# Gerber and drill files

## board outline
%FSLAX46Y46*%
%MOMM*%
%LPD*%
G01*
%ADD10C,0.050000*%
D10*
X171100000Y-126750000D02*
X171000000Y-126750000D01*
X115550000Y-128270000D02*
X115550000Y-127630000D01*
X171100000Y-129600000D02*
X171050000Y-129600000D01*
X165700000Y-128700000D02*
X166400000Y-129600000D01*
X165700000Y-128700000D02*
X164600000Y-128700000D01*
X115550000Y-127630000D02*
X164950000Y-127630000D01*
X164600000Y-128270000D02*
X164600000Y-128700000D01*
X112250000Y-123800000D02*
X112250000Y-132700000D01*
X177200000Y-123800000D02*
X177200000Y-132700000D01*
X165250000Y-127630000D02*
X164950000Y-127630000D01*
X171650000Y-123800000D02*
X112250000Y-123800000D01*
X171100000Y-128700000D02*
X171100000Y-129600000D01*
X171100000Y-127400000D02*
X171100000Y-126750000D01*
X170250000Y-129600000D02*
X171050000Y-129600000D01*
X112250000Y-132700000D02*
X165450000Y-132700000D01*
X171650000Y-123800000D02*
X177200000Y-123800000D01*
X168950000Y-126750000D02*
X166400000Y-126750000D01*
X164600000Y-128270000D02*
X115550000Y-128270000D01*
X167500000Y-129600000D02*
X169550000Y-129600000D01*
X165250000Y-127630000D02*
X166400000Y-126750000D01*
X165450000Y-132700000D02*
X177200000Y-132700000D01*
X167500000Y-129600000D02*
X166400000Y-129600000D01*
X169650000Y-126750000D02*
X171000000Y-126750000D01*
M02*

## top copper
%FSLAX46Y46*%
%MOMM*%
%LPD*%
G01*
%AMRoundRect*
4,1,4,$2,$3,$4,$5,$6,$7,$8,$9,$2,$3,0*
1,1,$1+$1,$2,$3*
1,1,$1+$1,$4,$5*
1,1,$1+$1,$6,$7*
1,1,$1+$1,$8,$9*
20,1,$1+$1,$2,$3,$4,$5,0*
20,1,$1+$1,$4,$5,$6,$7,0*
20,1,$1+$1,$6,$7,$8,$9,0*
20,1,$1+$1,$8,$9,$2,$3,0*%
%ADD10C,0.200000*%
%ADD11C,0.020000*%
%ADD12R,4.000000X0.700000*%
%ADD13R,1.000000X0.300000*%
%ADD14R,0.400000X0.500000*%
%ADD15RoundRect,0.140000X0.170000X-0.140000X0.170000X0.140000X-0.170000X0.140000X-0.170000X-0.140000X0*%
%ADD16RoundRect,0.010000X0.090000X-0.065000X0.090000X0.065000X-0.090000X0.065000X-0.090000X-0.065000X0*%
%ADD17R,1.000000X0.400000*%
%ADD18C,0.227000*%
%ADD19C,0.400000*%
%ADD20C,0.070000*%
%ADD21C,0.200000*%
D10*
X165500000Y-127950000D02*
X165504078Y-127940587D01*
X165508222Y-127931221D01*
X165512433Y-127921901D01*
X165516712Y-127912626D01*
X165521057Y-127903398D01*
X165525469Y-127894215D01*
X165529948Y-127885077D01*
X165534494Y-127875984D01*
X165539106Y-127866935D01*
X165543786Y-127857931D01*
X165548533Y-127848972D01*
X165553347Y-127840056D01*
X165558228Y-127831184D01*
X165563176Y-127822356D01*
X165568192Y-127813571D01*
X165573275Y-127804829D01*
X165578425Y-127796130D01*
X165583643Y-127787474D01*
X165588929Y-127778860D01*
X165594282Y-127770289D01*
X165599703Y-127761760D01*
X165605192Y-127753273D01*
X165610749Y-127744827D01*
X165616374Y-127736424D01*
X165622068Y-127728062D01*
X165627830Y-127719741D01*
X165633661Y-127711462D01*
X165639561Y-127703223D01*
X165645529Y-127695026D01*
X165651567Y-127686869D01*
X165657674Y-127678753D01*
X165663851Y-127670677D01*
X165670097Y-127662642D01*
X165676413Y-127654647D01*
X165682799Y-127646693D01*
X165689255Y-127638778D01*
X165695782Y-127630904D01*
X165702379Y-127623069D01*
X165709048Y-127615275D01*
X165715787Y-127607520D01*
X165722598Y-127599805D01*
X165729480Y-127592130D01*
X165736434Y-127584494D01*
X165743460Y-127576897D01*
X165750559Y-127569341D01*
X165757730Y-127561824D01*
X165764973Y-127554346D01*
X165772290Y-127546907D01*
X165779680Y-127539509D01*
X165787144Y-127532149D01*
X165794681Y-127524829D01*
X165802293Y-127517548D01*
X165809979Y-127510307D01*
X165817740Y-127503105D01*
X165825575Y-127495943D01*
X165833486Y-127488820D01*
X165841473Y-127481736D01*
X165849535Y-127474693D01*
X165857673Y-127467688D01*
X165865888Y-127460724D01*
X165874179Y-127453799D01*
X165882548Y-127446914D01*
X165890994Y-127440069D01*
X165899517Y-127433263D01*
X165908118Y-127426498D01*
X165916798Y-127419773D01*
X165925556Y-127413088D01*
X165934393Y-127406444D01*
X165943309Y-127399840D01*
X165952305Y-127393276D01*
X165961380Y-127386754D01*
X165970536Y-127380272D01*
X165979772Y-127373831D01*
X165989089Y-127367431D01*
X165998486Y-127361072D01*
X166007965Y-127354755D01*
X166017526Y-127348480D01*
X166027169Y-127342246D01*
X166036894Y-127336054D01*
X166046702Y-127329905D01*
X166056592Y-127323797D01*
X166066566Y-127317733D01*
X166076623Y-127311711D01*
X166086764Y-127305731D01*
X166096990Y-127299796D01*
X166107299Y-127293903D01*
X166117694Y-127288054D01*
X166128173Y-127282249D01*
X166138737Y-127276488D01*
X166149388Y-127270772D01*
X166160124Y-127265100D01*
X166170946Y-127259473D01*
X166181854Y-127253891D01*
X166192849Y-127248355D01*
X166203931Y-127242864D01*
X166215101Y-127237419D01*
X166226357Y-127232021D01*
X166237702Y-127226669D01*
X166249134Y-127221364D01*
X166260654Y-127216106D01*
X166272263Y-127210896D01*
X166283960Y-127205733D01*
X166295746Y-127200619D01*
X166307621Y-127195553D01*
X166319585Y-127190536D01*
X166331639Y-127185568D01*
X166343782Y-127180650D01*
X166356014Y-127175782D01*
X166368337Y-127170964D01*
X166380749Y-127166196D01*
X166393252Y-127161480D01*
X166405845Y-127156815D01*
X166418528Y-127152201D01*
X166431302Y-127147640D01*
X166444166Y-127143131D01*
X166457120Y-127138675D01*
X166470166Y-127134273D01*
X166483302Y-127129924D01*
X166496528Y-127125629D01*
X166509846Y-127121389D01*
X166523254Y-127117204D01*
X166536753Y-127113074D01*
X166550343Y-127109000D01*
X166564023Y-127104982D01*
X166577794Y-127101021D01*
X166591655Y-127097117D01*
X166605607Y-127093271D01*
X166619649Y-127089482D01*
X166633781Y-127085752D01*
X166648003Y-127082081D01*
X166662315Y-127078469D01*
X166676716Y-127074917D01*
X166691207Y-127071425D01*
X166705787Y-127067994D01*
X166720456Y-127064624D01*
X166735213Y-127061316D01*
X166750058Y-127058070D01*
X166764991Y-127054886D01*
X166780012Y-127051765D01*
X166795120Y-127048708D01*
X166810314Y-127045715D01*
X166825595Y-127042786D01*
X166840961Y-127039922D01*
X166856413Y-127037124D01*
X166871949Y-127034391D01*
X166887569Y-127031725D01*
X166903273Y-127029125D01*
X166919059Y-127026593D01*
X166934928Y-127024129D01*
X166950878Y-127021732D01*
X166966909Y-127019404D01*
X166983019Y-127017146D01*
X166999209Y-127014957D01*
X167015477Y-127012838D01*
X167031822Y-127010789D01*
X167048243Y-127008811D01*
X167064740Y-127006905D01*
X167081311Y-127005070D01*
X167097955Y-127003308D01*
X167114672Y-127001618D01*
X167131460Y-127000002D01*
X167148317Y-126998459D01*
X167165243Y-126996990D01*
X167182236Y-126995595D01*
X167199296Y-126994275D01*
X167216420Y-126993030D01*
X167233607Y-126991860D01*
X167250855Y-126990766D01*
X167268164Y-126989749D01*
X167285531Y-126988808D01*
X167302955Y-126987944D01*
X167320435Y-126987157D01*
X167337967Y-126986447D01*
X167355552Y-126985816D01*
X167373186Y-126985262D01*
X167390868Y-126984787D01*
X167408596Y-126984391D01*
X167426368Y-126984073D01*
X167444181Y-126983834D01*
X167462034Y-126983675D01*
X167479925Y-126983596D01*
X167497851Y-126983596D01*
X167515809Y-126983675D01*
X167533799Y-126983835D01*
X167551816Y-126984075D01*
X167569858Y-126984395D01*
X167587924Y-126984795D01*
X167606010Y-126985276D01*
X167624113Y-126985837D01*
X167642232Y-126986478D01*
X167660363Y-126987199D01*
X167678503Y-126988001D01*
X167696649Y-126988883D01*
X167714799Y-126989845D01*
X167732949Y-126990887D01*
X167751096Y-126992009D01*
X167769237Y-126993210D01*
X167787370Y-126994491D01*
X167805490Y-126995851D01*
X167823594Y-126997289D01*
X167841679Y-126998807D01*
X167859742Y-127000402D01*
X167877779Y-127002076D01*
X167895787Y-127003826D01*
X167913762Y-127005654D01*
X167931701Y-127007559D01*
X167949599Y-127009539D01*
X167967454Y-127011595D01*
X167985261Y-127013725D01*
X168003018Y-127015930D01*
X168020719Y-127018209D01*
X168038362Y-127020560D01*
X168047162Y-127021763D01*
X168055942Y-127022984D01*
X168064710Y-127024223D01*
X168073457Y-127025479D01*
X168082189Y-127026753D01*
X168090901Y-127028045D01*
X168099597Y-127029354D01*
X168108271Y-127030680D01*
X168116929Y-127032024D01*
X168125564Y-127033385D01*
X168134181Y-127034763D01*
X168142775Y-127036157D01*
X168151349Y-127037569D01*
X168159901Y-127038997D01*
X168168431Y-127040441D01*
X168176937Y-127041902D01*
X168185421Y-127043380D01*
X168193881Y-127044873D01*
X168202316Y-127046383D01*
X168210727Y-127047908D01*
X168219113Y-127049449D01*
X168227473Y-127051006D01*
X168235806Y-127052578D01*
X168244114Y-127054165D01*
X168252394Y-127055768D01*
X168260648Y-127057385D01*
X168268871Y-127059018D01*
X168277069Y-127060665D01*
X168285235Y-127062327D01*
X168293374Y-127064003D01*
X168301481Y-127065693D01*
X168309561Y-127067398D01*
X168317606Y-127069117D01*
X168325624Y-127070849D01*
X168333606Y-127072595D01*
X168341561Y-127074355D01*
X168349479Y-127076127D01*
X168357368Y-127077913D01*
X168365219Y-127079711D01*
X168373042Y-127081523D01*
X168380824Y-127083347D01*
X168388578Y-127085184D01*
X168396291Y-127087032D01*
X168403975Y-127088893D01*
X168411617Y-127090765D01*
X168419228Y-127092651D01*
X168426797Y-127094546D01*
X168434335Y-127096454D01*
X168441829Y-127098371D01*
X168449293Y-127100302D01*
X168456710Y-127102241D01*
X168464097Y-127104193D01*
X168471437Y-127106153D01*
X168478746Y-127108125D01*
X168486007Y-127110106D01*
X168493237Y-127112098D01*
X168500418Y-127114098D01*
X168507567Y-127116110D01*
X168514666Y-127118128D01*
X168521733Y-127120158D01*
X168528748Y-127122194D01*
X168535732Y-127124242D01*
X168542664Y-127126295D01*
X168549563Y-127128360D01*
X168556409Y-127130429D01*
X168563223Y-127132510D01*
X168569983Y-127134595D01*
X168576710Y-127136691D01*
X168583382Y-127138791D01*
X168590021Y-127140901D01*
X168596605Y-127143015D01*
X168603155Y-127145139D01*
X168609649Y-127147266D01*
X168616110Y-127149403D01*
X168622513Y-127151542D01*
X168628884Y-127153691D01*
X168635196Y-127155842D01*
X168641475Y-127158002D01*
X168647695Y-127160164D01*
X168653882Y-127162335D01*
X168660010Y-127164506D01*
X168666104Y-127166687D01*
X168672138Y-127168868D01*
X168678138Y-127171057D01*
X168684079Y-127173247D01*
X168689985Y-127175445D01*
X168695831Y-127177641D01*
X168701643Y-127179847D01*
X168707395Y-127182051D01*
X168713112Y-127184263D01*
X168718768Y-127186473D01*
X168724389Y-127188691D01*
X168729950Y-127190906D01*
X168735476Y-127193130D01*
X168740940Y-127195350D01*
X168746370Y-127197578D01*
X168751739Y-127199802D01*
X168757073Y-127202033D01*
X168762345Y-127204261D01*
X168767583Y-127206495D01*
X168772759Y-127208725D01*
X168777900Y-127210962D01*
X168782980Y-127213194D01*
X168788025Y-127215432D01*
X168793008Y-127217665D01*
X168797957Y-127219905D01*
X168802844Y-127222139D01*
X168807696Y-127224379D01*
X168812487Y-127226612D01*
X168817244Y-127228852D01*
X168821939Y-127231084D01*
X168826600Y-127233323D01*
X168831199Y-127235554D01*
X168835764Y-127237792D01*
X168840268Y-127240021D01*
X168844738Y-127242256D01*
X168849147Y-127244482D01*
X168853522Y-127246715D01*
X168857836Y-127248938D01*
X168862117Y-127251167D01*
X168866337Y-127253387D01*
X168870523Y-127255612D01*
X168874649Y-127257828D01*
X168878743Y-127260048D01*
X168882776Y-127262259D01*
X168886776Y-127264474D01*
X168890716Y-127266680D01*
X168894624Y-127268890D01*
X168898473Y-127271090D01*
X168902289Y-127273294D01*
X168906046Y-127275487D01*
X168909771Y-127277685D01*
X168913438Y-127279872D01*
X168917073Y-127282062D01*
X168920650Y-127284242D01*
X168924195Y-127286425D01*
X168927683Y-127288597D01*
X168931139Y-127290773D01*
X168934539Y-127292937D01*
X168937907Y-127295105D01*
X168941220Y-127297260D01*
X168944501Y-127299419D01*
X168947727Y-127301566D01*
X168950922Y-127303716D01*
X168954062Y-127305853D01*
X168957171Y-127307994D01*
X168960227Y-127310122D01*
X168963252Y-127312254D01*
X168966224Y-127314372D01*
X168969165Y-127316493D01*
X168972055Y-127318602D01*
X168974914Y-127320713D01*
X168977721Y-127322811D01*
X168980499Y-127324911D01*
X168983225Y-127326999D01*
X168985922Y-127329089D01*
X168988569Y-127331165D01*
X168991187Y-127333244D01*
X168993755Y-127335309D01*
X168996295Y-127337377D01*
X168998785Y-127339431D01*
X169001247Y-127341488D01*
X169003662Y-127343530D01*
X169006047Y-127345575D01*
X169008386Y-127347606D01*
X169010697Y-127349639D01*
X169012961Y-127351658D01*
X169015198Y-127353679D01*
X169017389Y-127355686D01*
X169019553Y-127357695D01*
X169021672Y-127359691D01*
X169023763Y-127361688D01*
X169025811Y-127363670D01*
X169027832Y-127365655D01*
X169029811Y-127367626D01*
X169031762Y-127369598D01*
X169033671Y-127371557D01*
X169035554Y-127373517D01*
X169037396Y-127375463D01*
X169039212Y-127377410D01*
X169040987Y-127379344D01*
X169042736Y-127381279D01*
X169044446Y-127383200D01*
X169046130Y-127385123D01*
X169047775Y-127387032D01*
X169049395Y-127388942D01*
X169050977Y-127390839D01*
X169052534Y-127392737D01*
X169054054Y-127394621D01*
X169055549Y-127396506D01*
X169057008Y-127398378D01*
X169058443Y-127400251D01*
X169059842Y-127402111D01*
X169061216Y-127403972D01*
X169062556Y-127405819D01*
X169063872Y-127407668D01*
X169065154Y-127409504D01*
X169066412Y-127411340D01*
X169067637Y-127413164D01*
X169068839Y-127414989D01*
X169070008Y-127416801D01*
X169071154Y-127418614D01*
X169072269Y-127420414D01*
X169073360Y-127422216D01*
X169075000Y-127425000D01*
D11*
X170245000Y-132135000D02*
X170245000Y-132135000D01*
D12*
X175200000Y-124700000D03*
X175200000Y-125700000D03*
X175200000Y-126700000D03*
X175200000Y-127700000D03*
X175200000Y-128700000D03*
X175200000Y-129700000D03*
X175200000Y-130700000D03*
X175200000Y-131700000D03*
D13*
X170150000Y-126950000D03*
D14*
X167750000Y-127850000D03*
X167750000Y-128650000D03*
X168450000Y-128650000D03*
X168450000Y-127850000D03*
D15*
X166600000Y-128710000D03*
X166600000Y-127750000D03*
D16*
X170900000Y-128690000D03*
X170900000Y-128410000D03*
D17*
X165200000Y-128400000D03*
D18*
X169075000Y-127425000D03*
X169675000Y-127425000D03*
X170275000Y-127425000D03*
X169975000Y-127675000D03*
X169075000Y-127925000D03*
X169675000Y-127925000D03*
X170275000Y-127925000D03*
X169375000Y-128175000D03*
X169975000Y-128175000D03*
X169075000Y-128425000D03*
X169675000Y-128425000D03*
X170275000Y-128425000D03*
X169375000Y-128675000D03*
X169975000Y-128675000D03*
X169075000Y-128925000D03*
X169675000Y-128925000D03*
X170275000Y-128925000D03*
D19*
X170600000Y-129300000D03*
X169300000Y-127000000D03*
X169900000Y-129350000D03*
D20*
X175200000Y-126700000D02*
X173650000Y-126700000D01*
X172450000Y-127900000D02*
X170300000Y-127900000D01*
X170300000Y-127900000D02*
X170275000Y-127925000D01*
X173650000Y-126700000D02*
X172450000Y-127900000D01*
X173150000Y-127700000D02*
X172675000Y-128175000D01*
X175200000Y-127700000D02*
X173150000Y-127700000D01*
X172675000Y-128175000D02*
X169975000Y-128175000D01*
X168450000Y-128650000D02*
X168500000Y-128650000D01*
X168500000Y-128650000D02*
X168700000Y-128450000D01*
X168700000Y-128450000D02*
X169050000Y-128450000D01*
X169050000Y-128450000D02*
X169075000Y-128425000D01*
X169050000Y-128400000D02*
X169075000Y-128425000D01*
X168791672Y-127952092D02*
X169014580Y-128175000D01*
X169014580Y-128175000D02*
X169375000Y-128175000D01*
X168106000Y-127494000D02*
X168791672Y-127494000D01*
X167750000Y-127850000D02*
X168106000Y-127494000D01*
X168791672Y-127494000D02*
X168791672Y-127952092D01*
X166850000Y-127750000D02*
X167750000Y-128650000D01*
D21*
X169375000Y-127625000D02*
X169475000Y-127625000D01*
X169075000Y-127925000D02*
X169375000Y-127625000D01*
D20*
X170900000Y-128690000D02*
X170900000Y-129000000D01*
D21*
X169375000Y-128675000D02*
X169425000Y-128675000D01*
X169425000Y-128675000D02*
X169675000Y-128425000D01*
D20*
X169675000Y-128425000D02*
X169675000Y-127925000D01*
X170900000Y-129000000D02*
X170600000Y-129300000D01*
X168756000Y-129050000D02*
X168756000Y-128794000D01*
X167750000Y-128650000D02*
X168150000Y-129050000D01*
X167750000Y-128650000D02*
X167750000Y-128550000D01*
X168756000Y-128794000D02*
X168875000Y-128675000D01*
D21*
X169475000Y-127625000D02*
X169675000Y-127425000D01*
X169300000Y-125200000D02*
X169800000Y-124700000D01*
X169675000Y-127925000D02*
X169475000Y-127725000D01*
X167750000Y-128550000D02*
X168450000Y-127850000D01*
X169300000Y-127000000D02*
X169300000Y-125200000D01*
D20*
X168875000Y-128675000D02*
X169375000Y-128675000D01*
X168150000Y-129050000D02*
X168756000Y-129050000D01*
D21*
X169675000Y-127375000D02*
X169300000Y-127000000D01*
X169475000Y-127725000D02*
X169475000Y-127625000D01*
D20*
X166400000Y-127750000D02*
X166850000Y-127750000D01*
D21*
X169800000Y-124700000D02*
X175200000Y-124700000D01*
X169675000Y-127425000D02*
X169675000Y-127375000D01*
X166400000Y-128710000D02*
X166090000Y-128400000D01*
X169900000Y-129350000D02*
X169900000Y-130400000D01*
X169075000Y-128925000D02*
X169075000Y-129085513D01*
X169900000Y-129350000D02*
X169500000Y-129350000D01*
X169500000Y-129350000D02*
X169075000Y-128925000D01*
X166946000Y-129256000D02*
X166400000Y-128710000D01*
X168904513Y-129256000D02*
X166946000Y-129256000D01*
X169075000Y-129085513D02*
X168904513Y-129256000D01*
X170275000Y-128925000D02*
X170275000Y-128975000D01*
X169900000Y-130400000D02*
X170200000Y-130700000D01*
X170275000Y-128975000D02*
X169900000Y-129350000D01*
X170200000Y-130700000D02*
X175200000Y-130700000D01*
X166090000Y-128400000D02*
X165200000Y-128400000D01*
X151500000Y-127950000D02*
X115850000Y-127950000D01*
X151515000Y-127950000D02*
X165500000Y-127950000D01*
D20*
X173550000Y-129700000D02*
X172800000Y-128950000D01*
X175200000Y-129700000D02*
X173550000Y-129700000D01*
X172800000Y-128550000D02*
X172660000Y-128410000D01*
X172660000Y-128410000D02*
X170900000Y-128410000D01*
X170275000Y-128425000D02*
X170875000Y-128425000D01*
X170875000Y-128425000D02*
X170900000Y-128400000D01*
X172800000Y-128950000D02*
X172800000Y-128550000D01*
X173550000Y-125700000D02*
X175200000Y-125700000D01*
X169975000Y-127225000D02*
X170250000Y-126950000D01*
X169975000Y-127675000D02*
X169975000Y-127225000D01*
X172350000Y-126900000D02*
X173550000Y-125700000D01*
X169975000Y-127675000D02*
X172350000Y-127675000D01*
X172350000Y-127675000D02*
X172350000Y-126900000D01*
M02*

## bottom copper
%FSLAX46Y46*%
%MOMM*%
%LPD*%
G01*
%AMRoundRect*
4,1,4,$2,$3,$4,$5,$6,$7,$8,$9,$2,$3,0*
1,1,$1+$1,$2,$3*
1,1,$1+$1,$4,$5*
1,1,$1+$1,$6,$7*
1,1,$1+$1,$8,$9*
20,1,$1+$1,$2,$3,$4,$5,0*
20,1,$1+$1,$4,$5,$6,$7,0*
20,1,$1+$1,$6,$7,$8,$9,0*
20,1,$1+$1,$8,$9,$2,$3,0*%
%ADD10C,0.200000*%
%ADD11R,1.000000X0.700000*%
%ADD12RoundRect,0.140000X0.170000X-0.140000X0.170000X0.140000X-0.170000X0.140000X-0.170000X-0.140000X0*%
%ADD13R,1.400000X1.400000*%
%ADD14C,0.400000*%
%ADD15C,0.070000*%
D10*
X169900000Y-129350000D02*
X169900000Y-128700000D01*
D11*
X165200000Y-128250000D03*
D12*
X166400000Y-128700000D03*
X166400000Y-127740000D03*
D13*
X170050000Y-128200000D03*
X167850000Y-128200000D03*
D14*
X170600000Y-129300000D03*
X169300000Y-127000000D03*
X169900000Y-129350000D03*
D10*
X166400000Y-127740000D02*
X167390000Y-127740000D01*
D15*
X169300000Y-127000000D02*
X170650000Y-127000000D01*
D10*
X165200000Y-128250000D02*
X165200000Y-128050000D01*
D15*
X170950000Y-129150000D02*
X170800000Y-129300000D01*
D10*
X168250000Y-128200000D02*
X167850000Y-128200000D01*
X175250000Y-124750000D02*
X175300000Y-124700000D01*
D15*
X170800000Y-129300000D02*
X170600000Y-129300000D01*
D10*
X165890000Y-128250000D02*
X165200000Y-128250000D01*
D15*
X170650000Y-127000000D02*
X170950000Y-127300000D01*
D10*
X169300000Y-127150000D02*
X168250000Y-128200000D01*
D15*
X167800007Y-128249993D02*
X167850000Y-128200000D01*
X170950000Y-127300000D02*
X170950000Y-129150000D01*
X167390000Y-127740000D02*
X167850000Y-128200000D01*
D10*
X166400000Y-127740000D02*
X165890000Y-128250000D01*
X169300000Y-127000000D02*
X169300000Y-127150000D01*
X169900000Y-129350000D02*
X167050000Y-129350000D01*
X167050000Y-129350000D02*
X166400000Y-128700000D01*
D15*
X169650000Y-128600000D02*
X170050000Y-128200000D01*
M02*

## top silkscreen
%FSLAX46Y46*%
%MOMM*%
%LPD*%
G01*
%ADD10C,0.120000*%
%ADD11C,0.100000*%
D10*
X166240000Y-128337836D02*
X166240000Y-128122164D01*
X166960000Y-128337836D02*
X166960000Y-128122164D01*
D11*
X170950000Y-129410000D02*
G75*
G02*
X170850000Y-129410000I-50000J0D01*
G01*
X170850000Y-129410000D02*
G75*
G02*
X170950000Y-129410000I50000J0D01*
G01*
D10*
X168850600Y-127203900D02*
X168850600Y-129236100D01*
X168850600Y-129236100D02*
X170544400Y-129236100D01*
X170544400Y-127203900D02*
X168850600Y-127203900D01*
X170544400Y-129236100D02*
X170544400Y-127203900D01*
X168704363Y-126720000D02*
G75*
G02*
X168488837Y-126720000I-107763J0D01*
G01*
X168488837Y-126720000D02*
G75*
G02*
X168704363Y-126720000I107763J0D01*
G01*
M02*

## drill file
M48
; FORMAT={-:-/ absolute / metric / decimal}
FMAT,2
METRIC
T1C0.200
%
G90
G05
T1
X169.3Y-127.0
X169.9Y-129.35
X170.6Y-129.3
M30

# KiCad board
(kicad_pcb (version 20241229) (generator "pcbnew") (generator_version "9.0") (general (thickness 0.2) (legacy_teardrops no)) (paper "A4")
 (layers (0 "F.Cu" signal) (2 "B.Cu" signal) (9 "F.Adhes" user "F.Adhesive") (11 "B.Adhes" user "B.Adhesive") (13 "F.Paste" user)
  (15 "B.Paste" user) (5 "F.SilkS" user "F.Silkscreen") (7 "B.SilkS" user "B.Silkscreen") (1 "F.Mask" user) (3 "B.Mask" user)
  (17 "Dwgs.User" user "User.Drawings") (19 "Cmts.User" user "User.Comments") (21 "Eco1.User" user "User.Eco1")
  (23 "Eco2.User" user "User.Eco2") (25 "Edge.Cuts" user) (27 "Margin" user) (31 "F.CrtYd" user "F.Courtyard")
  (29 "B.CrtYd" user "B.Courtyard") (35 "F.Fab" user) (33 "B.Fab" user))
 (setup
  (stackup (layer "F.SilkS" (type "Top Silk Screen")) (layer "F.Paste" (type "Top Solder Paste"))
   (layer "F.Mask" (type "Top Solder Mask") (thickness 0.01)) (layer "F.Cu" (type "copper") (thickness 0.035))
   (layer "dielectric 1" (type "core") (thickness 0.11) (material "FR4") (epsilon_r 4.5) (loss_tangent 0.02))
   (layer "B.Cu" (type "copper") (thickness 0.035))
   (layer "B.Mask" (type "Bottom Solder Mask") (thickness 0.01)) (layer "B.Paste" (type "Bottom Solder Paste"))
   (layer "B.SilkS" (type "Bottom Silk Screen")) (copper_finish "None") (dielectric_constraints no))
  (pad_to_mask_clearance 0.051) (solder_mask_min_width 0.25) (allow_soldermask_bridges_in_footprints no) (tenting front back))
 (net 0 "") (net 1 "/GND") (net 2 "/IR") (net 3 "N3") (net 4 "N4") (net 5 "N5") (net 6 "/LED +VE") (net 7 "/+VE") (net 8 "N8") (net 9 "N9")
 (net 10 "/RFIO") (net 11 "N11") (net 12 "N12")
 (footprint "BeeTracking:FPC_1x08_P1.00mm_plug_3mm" (layer "F.Cu") (at 173.2 128.2)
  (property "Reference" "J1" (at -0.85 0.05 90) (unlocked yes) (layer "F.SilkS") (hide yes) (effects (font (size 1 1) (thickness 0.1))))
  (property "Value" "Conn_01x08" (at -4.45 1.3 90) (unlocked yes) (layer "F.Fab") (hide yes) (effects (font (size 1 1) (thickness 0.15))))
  (pad "1" connect rect (at 2 -3.5) (size 4 0.7) (layers "F.Cu" "F.Mask") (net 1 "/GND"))
  (pad "2" connect rect (at 2 -2.5) (size 4 0.7) (layers "F.Cu" "F.Mask") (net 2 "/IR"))
  (pad "3" connect rect (at 2 -1.5) (size 4 0.7) (layers "F.Cu" "F.Mask") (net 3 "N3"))
  (pad "4" connect rect (at 2 -0.5) (size 4 0.7) (layers "F.Cu" "F.Mask") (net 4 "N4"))
  (pad "5" connect rect (at 2 0.5) (size 4 0.7) (layers "F.Cu" "F.Mask") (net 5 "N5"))
  (pad "6" connect rect (at 2 1.5) (size 4 0.7) (layers "F.Cu" "F.Mask") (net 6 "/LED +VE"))
  (pad "7" connect rect (at 2 2.5) (size 4 0.7) (layers "F.Cu" "F.Mask") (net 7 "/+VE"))
  (pad "8" connect rect (at 2 3.5) (size 4 0.7) (layers "F.Cu" "F.Mask")))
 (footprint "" (layer "F.Cu") (at 170.35 126.1)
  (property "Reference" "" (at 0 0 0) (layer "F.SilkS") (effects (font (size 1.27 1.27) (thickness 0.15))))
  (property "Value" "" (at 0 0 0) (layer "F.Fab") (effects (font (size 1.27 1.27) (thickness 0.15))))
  (pad "1" smd rect (at -0.2 0.85) (size 1 0.3) (layers "F.Cu" "F.Mask") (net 2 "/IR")))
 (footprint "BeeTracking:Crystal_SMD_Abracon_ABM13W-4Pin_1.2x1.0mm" (layer "F.Cu") (at 168.1 128.25 -90)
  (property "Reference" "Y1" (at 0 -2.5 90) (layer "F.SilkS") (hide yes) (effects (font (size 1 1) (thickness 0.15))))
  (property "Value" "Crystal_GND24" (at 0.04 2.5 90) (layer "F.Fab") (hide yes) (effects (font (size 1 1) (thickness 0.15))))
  (pad "1" smd rect (at -0.4 0.35 270) (size 0.5 0.4) (layers "F.Cu" "F.Mask" "F.Paste") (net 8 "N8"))
  (pad "2" smd rect (at 0.4 0.35 270) (size 0.5 0.4) (layers "F.Cu" "F.Mask" "F.Paste") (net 1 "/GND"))
  (pad "3" smd rect (at 0.4 -0.35 270) (size 0.5 0.4) (layers "F.Cu" "F.Mask" "F.Paste") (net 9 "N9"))
  (pad "4" smd rect (at -0.4 -0.35 270) (size 0.5 0.4) (layers "F.Cu" "F.Mask" "F.Paste") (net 1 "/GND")))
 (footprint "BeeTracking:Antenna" (layer "F.Cu") (at 170.245 132.135)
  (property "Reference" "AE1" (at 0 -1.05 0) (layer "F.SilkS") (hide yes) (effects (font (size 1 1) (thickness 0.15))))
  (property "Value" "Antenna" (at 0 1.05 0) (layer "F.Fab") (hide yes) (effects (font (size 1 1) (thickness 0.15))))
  (fp_line (start 0 0) (end 0 0) (stroke (width 0.02) (type solid)) (layer "F.Cu")))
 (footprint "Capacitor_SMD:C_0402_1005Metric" (layer "F.Cu") (at 166.6 128.23 90)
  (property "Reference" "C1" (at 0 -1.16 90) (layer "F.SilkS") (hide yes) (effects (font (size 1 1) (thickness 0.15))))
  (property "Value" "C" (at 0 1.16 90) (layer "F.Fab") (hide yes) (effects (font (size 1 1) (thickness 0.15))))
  (fp_line (start -0.107836 -0.36) (end 0.107836 -0.36) (stroke (width 0.12) (type solid)) (layer "F.SilkS"))
  (fp_line (start -0.107836 0.36) (end 0.107836 0.36) (stroke (width 0.12) (type solid)) (layer "F.SilkS"))
  (pad "1" smd roundrect (at -0.48 0 90) (size 0.56 0.62) (layers "F.Cu" "F.Mask" "F.Paste") (roundrect_rratio 0.25) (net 7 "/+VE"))
  (pad "2" smd roundrect (at 0.48 0 90) (size 0.56 0.62) (layers "F.Cu" "F.Mask" "F.Paste") (roundrect_rratio 0.25) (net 1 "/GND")))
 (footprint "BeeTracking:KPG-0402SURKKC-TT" (layer "F.Cu") (at 170.9 128.55 90)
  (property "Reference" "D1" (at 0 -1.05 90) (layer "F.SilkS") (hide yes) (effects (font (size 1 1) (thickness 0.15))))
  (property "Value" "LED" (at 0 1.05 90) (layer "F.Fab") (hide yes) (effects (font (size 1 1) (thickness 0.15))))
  (fp_circle (center -0.86 0) (end -0.81 0) (stroke (width 0.1) (type solid)) (fill no) (layer "F.SilkS"))
  (pad "" smd roundrect (at -0.14 0 90) (size 0.15 0.2) (layers "F.Mask") (roundrect_rratio 0.06666666667))
  (pad "" smd roundrect (at -0.1225 0 90) (size 0.1 0.17) (layers "F.Paste") (roundrect_rratio 0.25))
  (pad "" smd roundrect (at 0.1225 0 90) (size 0.1 0.17) (layers "F.Paste") (roundrect_rratio 0.25))
  (pad "" smd roundrect (at 0.14 0 90) (size 0.15 0.2) (layers "F.Mask") (roundrect_rratio 0.06666666667))
  (pad "1" smd roundrect (at -0.14 0 90) (size 0.15 0.2) (layers "F.Cu" "F.Mask") (roundrect_rratio 0.06666666667) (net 1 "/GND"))
  (pad "2" smd roundrect (at 0.14 0 90) (size 0.15 0.2) (layers "F.Cu" "F.Mask") (roundrect_rratio 0.06666666667) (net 6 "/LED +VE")))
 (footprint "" (layer "F.Cu") (at 165.4 127.6)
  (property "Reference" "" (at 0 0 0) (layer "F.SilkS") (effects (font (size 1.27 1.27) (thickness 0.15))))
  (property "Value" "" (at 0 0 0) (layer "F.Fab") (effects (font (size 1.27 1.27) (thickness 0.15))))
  (pad "1" smd rect (at -0.2 0.8) (size 1 0.4) (layers "F.Cu" "F.Mask") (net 7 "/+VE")))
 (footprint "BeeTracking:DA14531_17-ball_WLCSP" (layer "F.Cu") (at 169.697 128.22)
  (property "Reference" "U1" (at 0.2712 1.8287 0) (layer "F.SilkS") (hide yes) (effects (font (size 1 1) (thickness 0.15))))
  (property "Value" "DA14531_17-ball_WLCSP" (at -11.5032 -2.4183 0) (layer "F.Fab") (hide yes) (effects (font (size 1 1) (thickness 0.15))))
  (fp_line (start -0.8464 -1.0161) (end -0.8464 1.0161) (stroke (width 0.12) (type solid)) (layer "F.SilkS"))
  (fp_line (start -0.8464 1.0161) (end 0.8474 1.0161) (stroke (width 0.12) (type solid)) (layer "F.SilkS"))
  (fp_line (start 0.8474 -1.0161) (end -0.8464 -1.0161) (stroke (width 0.12) (type solid)) (layer "F.SilkS"))
  (fp_line (start 0.8474 1.0161) (end 0.8474 -1.0161) (stroke (width 0.12) (type solid)) (layer "F.SilkS"))
  (fp_circle (center -1.1004 -1.5) (end -1.0242 -1.4238) (stroke (width 0.12) (type solid)) (fill no) (layer "F.SilkS"))
  (pad "A1" smd circle (at -0.622 -0.795) (size 0.227 0.227) (layers "F.Cu" "F.Mask" "F.Paste") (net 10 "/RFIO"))
  (pad "A3" smd circle (at -0.022 -0.795) (size 0.227 0.227) (layers "F.Cu" "F.Mask" "F.Paste") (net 1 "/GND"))
  (pad "A5" smd circle (at 0.578 -0.795) (size 0.227 0.227) (layers "F.Cu" "F.Mask" "F.Paste") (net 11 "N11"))
  (pad "B4" smd circle (at 0.278 -0.545) (size 0.227 0.227) (layers "F.Cu" "F.Mask" "F.Paste") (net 2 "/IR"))
  (pad "C1" smd circle (at -0.622 -0.295) (size 0.227 0.227) (layers "F.Cu" "F.Mask" "F.Paste") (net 1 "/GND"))
  (pad "C3" smd circle (at -0.022 -0.295) (size 0.227 0.227) (layers "F.Cu" "F.Mask" "F.Paste") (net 1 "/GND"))
  (pad "C5" smd circle (at 0.578 -0.295) (size 0.227 0.227) (layers "F.Cu" "F.Mask" "F.Paste") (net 3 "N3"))
  (pad "D2" smd circle (at -0.322 -0.045) (size 0.227 0.227) (layers "F.Cu" "F.Mask" "F.Paste") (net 8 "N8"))
  (pad "D4" smd circle (at 0.278 -0.045) (size 0.227 0.227) (layers "F.Cu" "F.Mask" "F.Paste") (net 4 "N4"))
  (pad "E1" smd circle (at -0.622 0.205) (size 0.227 0.227) (layers "F.Cu" "F.Mask" "F.Paste") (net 9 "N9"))
  (pad "E3" smd circle (at -0.022 0.205) (size 0.227 0.227) (layers "F.Cu" "F.Mask" "F.Paste") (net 1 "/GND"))
  (pad "E5" smd circle (at 0.578 0.205) (size 0.227 0.227) (layers "F.Cu" "F.Mask" "F.Paste") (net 6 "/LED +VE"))
  (pad "F2" smd circle (at -0.322 0.455) (size 0.227 0.227) (layers "F.Cu" "F.Mask" "F.Paste") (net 1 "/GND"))
  (pad "F4" smd circle (at 0.278 0.455) (size 0.227 0.227) (layers "F.Cu" "F.Mask" "F.Paste") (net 5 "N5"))
  (pad "G1" smd circle (at -0.622 0.705) (size 0.227 0.227) (layers "F.Cu" "F.Mask" "F.Paste") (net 7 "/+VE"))
  (pad "G3" smd circle (at -0.022 0.705) (size 0.227 0.227) (layers "F.Cu" "F.Mask" "F.Paste") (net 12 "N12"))
  (pad "G5" smd circle (at 0.578 0.705) (size 0.227 0.227) (layers "F.Cu" "F.Mask" "F.Paste") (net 7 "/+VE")))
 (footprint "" (layer "B.Cu") (at 165.2 128.4 180)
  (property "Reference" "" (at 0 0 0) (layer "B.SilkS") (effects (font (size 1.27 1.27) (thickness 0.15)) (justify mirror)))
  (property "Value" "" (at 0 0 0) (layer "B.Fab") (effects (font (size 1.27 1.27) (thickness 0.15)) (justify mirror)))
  (pad "1" smd rect (at 0 0.15 180) (size 1 0.7) (layers "B.Cu" "B.Mask") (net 1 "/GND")))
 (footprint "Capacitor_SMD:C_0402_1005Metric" (layer "B.Cu") (at 166.4 128.22 90)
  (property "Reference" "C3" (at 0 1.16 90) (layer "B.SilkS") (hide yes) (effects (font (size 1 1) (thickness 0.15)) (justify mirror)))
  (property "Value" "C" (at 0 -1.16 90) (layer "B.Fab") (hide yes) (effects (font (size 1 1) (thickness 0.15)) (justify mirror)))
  (pad "1" smd roundrect (at -0.48 0 90) (size 0.56 0.62) (layers "B.Cu" "B.Mask" "B.Paste") (roundrect_rratio 0.25) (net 7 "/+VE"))
  (pad "2" smd roundrect (at 0.48 0 90) (size 0.56 0.62) (layers "B.Cu" "B.Mask" "B.Paste") (roundrect_rratio 0.25) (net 1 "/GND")))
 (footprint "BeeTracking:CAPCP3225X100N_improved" (layer "B.Cu") (at 168.95 128.2 180)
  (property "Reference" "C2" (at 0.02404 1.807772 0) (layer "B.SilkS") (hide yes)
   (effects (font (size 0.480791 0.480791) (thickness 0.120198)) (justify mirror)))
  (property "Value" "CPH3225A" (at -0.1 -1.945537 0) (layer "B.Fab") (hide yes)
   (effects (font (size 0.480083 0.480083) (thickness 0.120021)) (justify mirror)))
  (pad "1" smd rect (at -1.1 0) (size 1.4 1.4) (layers "B.Cu" "B.Mask" "B.Paste") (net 7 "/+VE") (solder_mask_margin 0.102))
  (pad "2" smd rect (at 1.1 0) (size 1.4 1.4) (layers "B.Cu" "B.Mask" "B.Paste") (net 1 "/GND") (solder_mask_margin 0.102)))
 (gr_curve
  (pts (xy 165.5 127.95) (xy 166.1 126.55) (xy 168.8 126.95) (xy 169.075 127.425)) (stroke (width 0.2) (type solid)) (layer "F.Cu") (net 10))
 (gr_line (start 169.9 129.35) (end 169.9 128.7) (stroke (width 0.2) (type default)) (layer "B.Cu") (net 7))
 (gr_line (start 171.1 126.75) (end 171 126.75) (stroke (width 0.05) (type default)) (layer "Edge.Cuts"))
 (gr_line (start 115.55 128.27) (end 115.55 127.63) (stroke (width 0.05) (type default)) (layer "Edge.Cuts"))
 (gr_line (start 171.1 129.6) (end 171.05 129.6) (stroke (width 0.05) (type default)) (layer "Edge.Cuts"))
 (gr_line (start 165.7 128.7) (end 166.4 129.6) (stroke (width 0.05) (type default)) (layer "Edge.Cuts"))
 (gr_line (start 165.7 128.7) (end 164.6 128.7) (stroke (width 0.05) (type default)) (layer "Edge.Cuts"))
 (gr_line (start 115.55 127.63) (end 164.95 127.63) (stroke (width 0.05) (type default)) (layer "Edge.Cuts"))
 (gr_line (start 164.6 128.27) (end 164.6 128.7) (stroke (width 0.05) (type default)) (layer "Edge.Cuts"))
 (gr_line (start 112.25 123.8) (end 112.25 132.7) (stroke (width 0.05) (type default)) (layer "Edge.Cuts"))
 (gr_line (start 177.2 123.8) (end 177.2 132.7) (stroke (width 0.05) (type default)) (layer "Edge.Cuts"))
 (gr_line (start 165.25 127.63) (end 164.95 127.63) (stroke (width 0.05) (type default)) (layer "Edge.Cuts"))
 (gr_line (start 171.65 123.8) (end 112.25 123.8) (stroke (width 0.05) (type default)) (layer "Edge.Cuts"))
 (gr_line (start 171.1 128.7) (end 171.1 129.6) (stroke (width 0.05) (type default)) (layer "Edge.Cuts"))
 (gr_line (start 171.1 127.4) (end 171.1 126.75) (stroke (width 0.05) (type default)) (layer "Edge.Cuts"))
 (gr_line (start 170.25 129.6) (end 171.05 129.6) (stroke (width 0.05) (type default)) (layer "Edge.Cuts"))
 (gr_line (start 112.25 132.7) (end 165.45 132.7) (stroke (width 0.05) (type default)) (layer "Edge.Cuts"))
 (gr_line (start 171.65 123.8) (end 177.2 123.8) (stroke (width 0.05) (type default)) (layer "Edge.Cuts"))
 (gr_line (start 168.95 126.75) (end 166.4 126.75) (stroke (width 0.05) (type default)) (layer "Edge.Cuts"))
 (gr_line (start 164.6 128.27) (end 115.55 128.27) (stroke (width 0.05) (type default)) (layer "Edge.Cuts"))
 (gr_line (start 167.5 129.6) (end 169.55 129.6) (stroke (width 0.05) (type default)) (layer "Edge.Cuts"))
 (gr_line (start 165.25 127.63) (end 166.4 126.75) (stroke (width 0.05) (type default)) (layer "Edge.Cuts"))
 (gr_line (start 165.45 132.7) (end 177.2 132.7) (stroke (width 0.05) (type default)) (layer "Edge.Cuts"))
 (gr_line (start 167.5 129.6) (end 166.4 129.6) (stroke (width 0.05) (type default)) (layer "Edge.Cuts"))
 (gr_line (start 169.65 126.75) (end 171 126.75) (stroke (width 0.05) (type default)) (layer "Edge.Cuts"))
 (segment (start 175.2 126.7) (end 173.65 126.7) (width 0.07) (layer "F.Cu") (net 3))
 (segment (start 172.45 127.9) (end 170.3 127.9) (width 0.07) (layer "F.Cu") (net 3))
 (segment (start 170.3 127.9) (end 170.275 127.925) (width 0.07) (layer "F.Cu") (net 3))
 (segment (start 173.65 126.7) (end 172.45 127.9) (width 0.07) (layer "F.Cu") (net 3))
 (segment (start 173.15 127.7) (end 172.675 128.175) (width 0.07) (layer "F.Cu") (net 4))
 (segment (start 175.2 127.7) (end 173.15 127.7) (width 0.07) (layer "F.Cu") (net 4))
 (segment (start 172.675 128.175) (end 169.975 128.175) (width 0.07) (layer "F.Cu") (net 4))
 (segment (start 168.45 128.65) (end 168.5 128.65) (width 0.07) (layer "F.Cu") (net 9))
 (segment (start 168.5 128.65) (end 168.7 128.45) (width 0.07) (layer "F.Cu") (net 9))
 (segment (start 168.7 128.45) (end 169.05 128.45) (width 0.07) (layer "F.Cu") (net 9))
 (segment (start 169.05 128.45) (end 169.075 128.425) (width 0.07) (layer "F.Cu") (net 9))
 (segment (start 169.05 128.4) (end 169.075 128.425) (width 0.07) (layer "F.Cu") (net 9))
 (segment (start 168.791672 127.952092) (end 169.01458 128.175) (width 0.07) (layer "F.Cu") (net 8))
 (segment (start 169.01458 128.175) (end 169.375 128.175) (width 0.07) (layer "F.Cu") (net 8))
 (segment (start 168.106 127.494) (end 168.791672 127.494) (width 0.07) (layer "F.Cu") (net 8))
 (segment (start 167.75 127.85) (end 168.106 127.494) (width 0.07) (layer "F.Cu") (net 8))
 (segment (start 168.791672 127.494) (end 168.791672 127.952092) (width 0.07) (layer "F.Cu") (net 8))
 (segment (start 166.85 127.75) (end 167.75 128.65) (width 0.07) (layer "F.Cu") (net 1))
 (segment (start 169.375 127.625) (end 169.475 127.625) (width 0.2) (layer "F.Cu") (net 1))
 (segment (start 169.075 127.925) (end 169.375 127.625) (width 0.2) (layer "F.Cu") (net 1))
 (segment (start 170.9 128.69) (end 170.9 129) (width 0.07) (layer "F.Cu") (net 1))
 (segment (start 169.375 128.675) (end 169.425 128.675) (width 0.2) (layer "F.Cu") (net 1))
 (segment (start 169.425 128.675) (end 169.675 128.425) (width 0.2) (layer "F.Cu") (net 1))
 (segment (start 169.675 128.425) (end 169.675 127.925) (width 0.07) (layer "F.Cu") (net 1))
 (segment (start 170.9 129) (end 170.6 129.3) (width 0.07) (layer "F.Cu") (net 1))
 (segment (start 168.756 129.05) (end 168.756 128.794) (width 0.07) (layer "F.Cu") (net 1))
 (segment (start 167.75 128.65) (end 168.15 129.05) (width 0.07) (layer "F.Cu") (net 1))
 (segment (start 167.75 128.65) (end 167.75 128.55) (width 0.07) (layer "F.Cu") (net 1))
 (segment (start 168.756 128.794) (end 168.875 128.675) (width 0.07) (layer "F.Cu") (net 1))
 (segment (start 169.475 127.625) (end 169.675 127.425) (width 0.2) (layer "F.Cu") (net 1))
 (segment (start 169.3 125.2) (end 169.8 124.7) (width 0.2) (layer "F.Cu") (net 1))
 (segment (start 169.675 127.925) (end 169.475 127.725) (width 0.2) (layer "F.Cu") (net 1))
 (segment (start 167.75 128.55) (end 168.45 127.85) (width 0.2) (layer "F.Cu") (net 1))
 (segment (start 169.3 127) (end 169.3 125.2) (width 0.2) (layer "F.Cu") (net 1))
 (segment (start 168.875 128.675) (end 169.375 128.675) (width 0.07) (layer "F.Cu") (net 1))
 (segment (start 168.15 129.05) (end 168.756 129.05) (width 0.07) (layer "F.Cu") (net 1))
 (segment (start 169.675 127.375) (end 169.3 127) (width 0.2) (layer "F.Cu") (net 1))
 (segment (start 169.475 127.725) (end 169.475 127.625) (width 0.2) (layer "F.Cu") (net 1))
 (segment (start 166.4 127.75) (end 166.85 127.75) (width 0.07) (layer "F.Cu") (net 1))
 (segment (start 169.8 124.7) (end 175.2 124.7) (width 0.2) (layer "F.Cu") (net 1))
 (segment (start 169.675 127.425) (end 169.675 127.375) (width 0.2) (layer "F.Cu") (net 1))
 (via (at 170.6 129.3) (size 0.4) (drill 0.2) (layers "F.Cu" "B.Cu") (free yes) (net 1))
 (via (at 169.3 127) (size 0.4) (drill 0.2) (layers "F.Cu" "B.Cu") (free yes) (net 1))
 (segment (start 166.4 127.74) (end 167.39 127.74) (width 0.2) (layer "B.Cu") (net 1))
 (segment (start 169.3 127) (end 170.65 127) (width 0.07) (layer "B.Cu") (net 1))
 (segment (start 165.2 128.25) (end 165.2 128.05) (width 0.2) (layer "B.Cu") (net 1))
 (segment (start 170.95 129.15) (end 170.8 129.3) (width 0.07) (layer "B.Cu") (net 1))
 (segment (start 168.25 128.2) (end 167.85 128.2) (width 0.2) (layer "B.Cu") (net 1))
 (segment (start 175.25 124.75) (end 175.3 124.7) (width 0.2) (layer "B.Cu") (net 1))
 (segment (start 170.8 129.3) (end 170.6 129.3) (width 0.07) (layer "B.Cu") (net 1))
 (segment (start 165.89 128.25) (end 165.2 128.25) (width 0.2) (layer "B.Cu") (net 1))
 (segment (start 170.65 127) (end 170.95 127.3) (width 0.07) (layer "B.Cu") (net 1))
 (segment (start 169.3 127.15) (end 168.25 128.2) (width 0.2) (layer "B.Cu") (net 1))
 (segment (start 167.800007 128.249993) (end 167.85 128.2) (width 0.07) (layer "B.Cu") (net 1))
 (segment (start 170.95 127.3) (end 170.95 129.15) (width 0.07) (layer "B.Cu") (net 1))
 (segment (start 167.39 127.74) (end 167.85 128.2) (width 0.07) (layer "B.Cu") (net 1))
 (segment (start 166.4 127.74) (end 165.89 128.25) (width 0.2) (layer "B.Cu") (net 1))
 (segment (start 169.3 127) (end 169.3 127.15) (width 0.2) (layer "B.Cu") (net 1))
 (segment (start 166.4 128.71) (end 166.09 128.4) (width 0.2) (layer "F.Cu") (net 7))
 (segment (start 169.9 129.35) (end 169.9 130.4) (width 0.2) (layer "F.Cu") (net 7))
 (segment (start 169.075 128.925) (end 169.075 129.085513) (width 0.2) (layer "F.Cu") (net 7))
 (segment (start 169.9 129.35) (end 169.5 129.35) (width 0.2) (layer "F.Cu") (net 7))
 (segment (start 169.5 129.35) (end 169.075 128.925) (width 0.2) (layer "F.Cu") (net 7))
 (segment (start 166.946 129.256) (end 166.4 128.71) (width 0.2) (layer "F.Cu") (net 7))
 (segment (start 168.904513 129.256) (end 166.946 129.256) (width 0.2) (layer "F.Cu") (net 7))
 (segment (start 169.075 129.085513) (end 168.904513 129.256) (width 0.2) (layer "F.Cu") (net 7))
 (segment (start 170.275 128.925) (end 170.275 128.975) (width 0.2) (layer "F.Cu") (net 7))
 (segment (start 169.9 130.4) (end 170.2 130.7) (width 0.2) (layer "F.Cu") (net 7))
 (segment (start 170.275 128.975) (end 169.9 129.35) (width 0.2) (layer "F.Cu") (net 7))
 (segment (start 170.2 130.7) (end 175.2 130.7) (width 0.2) (layer "F.Cu") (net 7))
 (segment (start 166.09 128.4) (end 165.2 128.4) (width 0.2) (layer "F.Cu") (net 7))
 (via (at 169.9 129.35) (size 0.4) (drill 0.2) (layers "F.Cu" "B.Cu") (free yes) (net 7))
 (segment (start 169.9 129.35) (end 167.05 129.35) (width 0.2) (layer "B.Cu") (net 7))
 (segment (start 167.05 129.35) (end 166.4 128.7) (width 0.2) (layer "B.Cu") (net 7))
 (segment (start 169.65 128.6) (end 170.05 128.2) (width 0.07) (layer "B.Cu") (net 7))
 (segment (start 151.5 127.95) (end 115.85 127.95) (width 0.2) (layer "F.Cu") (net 10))
 (segment (start 151.515 127.95) (end 165.5 127.95) (width 0.2) (layer "F.Cu") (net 10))
 (segment (start 173.55 129.7) (end 172.8 128.95) (width 0.07) (layer "F.Cu") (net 6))
 (segment (start 175.2 129.7) (end 173.55 129.7) (width 0.07) (layer "F.Cu") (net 6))
 (segment (start 172.8 128.55) (end 172.66 128.41) (width 0.07) (layer "F.Cu") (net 6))
 (segment (start 172.66 128.41) (end 170.9 128.41) (width 0.07) (layer "F.Cu") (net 6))
 (segment (start 170.275 128.425) (end 170.875 128.425) (width 0.07) (layer "F.Cu") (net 6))
 (segment (start 170.875 128.425) (end 170.9 128.4) (width 0.07) (layer "F.Cu") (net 6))
 (segment (start 172.8 128.95) (end 172.8 128.55) (width 0.07) (layer "F.Cu") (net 6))
 (segment (start 173.55 125.7) (end 175.2 125.7) (width 0.07) (layer "F.Cu") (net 2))
 (segment (start 169.975 127.225) (end 170.25 126.95) (width 0.07) (layer "F.Cu") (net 2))
 (segment (start 169.975 127.675) (end 169.975 127.225) (width 0.07) (layer "F.Cu") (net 2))
 (segment (start 172.35 126.9) (end 173.55 125.7) (width 0.07) (layer "F.Cu") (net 2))
 (segment (start 169.975 127.675) (end 172.35 127.675) (width 0.07) (layer "F.Cu") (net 2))
 (segment (start 172.35 127.675) (end 172.35 126.9) (width 0.07) (layer "F.Cu") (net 2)))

